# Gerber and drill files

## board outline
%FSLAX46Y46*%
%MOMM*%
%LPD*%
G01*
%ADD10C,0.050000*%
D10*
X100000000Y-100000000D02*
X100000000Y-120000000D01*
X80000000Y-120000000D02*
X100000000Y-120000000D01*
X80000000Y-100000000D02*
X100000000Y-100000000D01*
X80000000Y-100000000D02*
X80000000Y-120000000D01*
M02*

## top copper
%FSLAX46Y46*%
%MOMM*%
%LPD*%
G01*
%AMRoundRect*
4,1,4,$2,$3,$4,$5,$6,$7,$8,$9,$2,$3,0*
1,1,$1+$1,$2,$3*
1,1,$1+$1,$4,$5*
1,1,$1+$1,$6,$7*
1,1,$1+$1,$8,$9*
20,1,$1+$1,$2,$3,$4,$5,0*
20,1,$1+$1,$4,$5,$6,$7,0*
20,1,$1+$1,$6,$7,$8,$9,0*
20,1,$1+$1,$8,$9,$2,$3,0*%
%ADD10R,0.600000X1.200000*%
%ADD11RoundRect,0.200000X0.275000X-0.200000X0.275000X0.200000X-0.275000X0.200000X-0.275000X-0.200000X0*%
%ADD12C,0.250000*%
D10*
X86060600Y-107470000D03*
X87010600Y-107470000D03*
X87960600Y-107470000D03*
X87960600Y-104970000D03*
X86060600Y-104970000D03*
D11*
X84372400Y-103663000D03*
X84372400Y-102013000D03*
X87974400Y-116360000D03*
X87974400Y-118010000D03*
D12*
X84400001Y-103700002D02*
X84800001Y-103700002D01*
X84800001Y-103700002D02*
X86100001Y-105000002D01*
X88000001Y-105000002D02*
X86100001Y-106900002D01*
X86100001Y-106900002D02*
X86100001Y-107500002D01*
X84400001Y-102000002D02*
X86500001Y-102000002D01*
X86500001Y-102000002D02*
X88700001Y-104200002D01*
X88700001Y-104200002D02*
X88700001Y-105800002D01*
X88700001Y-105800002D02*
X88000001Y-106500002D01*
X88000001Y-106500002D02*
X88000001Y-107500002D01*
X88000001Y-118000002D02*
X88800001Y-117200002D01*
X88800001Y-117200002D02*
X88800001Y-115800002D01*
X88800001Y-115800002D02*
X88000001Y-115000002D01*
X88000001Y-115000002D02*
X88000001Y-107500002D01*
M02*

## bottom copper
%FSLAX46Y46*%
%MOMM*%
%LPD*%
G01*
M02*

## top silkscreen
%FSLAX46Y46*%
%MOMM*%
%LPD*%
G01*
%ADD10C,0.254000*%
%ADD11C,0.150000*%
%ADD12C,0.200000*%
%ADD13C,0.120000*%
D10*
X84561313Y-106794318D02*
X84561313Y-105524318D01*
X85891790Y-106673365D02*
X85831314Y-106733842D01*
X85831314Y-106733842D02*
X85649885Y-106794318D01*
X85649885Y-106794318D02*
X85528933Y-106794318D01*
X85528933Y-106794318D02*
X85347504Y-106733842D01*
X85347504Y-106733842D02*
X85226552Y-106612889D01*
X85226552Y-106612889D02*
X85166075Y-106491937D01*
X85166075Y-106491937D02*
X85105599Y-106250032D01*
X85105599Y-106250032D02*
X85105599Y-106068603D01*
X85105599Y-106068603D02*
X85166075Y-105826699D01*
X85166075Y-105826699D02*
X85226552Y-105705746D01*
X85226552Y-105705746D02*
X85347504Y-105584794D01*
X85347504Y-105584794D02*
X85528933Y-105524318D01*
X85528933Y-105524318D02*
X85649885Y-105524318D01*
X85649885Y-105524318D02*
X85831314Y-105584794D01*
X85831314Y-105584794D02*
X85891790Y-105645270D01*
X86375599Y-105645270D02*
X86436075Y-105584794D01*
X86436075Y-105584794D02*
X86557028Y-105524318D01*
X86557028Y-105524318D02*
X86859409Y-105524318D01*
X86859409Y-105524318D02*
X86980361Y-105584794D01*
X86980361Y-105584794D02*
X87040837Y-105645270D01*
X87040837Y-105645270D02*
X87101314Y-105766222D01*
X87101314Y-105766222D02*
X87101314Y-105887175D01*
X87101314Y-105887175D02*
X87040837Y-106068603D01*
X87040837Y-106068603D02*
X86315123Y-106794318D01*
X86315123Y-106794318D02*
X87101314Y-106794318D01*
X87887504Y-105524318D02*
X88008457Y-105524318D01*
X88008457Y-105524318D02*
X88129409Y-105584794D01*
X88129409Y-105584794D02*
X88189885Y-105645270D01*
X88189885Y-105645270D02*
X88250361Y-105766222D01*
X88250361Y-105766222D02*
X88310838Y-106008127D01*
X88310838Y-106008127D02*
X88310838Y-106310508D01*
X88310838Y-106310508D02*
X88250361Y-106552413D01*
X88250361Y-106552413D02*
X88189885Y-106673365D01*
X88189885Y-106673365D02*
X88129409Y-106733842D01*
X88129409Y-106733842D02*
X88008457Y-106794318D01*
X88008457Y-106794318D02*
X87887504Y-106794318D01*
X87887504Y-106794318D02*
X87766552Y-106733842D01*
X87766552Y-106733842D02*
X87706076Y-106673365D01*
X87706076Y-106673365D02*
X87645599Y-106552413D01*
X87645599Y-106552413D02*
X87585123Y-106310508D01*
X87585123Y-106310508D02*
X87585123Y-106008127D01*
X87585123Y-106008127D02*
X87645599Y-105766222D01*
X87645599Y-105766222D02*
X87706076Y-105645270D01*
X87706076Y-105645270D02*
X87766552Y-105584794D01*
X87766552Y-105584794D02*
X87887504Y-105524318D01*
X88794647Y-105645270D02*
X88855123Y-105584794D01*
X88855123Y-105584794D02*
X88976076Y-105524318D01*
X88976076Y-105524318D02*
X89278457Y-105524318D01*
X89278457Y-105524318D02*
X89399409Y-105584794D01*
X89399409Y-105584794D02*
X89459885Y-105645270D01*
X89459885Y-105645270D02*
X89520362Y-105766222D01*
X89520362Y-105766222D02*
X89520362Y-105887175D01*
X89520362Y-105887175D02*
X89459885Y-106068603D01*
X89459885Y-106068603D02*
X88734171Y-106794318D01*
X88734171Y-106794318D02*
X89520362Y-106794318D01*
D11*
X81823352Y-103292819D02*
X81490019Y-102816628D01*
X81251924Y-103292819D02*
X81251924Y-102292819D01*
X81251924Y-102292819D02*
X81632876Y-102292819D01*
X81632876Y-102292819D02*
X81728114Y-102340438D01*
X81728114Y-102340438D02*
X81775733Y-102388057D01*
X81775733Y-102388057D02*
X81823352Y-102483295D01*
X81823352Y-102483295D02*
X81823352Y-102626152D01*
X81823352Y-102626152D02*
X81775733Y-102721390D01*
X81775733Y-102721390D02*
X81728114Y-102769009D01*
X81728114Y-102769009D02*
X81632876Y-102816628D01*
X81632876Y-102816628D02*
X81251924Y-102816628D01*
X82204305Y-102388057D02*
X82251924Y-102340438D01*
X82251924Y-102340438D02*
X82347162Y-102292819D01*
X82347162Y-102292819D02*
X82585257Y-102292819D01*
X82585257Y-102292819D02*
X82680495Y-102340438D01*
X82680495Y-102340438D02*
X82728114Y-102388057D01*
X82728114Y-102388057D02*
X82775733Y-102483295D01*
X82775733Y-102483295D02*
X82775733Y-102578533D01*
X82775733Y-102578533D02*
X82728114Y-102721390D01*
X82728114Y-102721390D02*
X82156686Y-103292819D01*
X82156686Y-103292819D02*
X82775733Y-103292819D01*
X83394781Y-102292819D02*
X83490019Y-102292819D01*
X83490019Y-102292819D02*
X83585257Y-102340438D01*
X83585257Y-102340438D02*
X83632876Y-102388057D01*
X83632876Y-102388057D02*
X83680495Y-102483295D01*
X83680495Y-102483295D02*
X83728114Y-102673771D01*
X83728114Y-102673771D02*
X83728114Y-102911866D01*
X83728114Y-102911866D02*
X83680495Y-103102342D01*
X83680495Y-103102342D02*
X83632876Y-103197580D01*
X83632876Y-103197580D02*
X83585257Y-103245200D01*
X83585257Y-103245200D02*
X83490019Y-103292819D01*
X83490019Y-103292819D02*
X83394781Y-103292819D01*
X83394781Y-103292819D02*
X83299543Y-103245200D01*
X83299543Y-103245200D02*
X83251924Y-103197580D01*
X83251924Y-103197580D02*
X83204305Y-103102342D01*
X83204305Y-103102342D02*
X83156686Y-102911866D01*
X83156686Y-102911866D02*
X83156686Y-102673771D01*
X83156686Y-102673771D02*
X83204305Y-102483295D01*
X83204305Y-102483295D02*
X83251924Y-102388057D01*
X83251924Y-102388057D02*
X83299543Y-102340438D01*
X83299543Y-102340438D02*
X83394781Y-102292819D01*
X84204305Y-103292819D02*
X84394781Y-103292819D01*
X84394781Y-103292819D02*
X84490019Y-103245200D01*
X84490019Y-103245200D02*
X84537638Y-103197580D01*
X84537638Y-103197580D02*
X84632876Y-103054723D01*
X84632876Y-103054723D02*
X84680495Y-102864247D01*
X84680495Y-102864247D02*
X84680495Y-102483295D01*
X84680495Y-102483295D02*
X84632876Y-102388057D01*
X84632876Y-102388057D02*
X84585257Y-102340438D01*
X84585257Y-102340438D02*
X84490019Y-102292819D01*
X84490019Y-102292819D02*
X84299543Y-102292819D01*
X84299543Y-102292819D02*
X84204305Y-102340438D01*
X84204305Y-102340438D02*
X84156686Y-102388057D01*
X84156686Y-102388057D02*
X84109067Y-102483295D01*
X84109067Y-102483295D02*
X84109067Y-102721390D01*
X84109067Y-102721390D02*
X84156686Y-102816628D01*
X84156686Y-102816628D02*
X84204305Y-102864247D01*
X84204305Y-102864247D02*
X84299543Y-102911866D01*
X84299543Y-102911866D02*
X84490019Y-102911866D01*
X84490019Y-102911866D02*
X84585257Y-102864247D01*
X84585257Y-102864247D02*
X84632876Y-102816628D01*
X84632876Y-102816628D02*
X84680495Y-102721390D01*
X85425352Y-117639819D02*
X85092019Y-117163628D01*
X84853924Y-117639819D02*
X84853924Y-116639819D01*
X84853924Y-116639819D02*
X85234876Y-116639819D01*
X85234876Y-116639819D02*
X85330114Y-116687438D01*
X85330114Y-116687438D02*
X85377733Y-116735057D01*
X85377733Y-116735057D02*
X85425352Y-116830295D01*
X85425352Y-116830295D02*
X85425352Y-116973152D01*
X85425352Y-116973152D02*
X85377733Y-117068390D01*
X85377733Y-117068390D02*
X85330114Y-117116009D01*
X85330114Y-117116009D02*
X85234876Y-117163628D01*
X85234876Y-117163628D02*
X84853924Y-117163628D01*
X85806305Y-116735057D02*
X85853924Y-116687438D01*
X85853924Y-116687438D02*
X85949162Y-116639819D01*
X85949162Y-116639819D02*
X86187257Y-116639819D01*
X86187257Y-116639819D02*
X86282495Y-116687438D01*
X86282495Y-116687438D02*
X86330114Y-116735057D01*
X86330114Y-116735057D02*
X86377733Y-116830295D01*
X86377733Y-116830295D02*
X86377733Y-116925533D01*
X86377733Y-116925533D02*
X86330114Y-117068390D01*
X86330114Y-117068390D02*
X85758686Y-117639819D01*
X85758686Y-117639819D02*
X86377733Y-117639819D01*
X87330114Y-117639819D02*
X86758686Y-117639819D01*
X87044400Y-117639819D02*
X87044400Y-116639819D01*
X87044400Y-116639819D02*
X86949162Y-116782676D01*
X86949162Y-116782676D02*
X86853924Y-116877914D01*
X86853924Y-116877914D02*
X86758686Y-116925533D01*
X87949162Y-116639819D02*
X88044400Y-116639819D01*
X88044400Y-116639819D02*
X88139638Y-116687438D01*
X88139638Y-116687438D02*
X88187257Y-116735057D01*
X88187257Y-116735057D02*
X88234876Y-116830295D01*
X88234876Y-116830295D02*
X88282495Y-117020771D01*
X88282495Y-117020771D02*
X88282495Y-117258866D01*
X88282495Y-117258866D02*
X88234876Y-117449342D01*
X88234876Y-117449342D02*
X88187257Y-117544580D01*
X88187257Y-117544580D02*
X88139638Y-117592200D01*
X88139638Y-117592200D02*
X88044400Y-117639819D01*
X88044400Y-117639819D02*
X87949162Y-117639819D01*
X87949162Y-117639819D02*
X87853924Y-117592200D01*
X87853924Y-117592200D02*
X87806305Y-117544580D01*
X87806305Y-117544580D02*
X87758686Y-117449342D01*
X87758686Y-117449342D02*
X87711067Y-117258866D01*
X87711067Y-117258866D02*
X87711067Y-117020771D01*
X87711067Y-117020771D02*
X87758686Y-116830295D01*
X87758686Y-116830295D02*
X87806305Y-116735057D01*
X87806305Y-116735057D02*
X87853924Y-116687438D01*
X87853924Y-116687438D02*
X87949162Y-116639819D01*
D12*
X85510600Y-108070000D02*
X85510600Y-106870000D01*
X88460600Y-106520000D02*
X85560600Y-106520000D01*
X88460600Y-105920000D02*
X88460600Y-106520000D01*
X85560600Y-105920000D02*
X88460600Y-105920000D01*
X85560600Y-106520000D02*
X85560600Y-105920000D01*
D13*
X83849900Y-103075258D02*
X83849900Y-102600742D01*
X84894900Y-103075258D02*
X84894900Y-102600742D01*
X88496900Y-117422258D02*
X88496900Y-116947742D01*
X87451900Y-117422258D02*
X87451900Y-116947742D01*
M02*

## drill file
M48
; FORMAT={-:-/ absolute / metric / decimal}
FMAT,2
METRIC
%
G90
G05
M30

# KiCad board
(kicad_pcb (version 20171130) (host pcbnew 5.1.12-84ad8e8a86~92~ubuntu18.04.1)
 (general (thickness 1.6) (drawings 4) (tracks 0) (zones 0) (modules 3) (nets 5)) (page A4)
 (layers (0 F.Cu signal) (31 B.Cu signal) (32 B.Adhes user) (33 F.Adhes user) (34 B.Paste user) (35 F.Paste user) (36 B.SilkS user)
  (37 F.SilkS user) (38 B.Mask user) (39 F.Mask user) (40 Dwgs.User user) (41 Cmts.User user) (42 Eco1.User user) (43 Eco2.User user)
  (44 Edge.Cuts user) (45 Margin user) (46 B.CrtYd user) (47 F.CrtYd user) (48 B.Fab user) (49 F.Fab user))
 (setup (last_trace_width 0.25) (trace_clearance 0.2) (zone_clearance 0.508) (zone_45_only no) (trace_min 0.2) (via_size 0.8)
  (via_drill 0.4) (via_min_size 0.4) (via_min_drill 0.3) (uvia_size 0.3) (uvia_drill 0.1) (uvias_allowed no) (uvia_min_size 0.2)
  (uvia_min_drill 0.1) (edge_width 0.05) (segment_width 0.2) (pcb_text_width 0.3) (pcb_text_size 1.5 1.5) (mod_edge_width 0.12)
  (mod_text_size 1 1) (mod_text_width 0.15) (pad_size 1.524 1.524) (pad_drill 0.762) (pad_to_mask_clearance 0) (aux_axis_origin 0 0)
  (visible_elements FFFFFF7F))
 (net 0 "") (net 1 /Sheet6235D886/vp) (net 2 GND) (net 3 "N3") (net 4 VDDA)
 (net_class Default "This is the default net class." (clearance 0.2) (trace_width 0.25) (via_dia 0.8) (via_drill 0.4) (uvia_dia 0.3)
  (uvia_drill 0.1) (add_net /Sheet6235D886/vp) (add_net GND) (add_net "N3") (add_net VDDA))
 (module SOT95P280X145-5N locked (layer F.Cu) (at 87.010600 106.220000 90.000000)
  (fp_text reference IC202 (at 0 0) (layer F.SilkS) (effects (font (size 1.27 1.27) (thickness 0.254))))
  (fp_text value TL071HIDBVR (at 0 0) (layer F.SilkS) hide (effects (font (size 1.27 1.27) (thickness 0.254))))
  (fp_line (start -1.85 -1.5) (end -0.65 -1.5) (layer F.SilkS) (width 0.2))
  (fp_line (start -0.3 1.45) (end -0.3 -1.45) (layer F.SilkS) (width 0.2))
  (fp_line (start 0.3 1.45) (end -0.3 1.45) (layer F.SilkS) (width 0.2))
  (fp_line (start 0.3 -1.45) (end 0.3 1.45) (layer F.SilkS) (width 0.2))
  (fp_line (start -0.3 -1.45) (end 0.3 -1.45) (layer F.SilkS) (width 0.2))
  (pad 1 smd rect (at -1.25 -0.95 180.000000) (size 0.6 1.2) (layers F.Cu F.Mask F.Paste) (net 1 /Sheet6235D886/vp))
  (pad 2 smd rect (at -1.25 0 180.000000) (size 0.6 1.2) (layers F.Cu F.Mask F.Paste) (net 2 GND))
  (pad 3 smd rect (at -1.25 0.95 180.000000) (size 0.6 1.2) (layers F.Cu F.Mask F.Paste) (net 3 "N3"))
  (pad 4 smd rect (at 1.25 0.95 180.000000) (size 0.6 1.2) (layers F.Cu F.Mask F.Paste) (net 1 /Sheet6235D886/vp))
  (pad 5 smd rect (at 1.25 -0.95 180.000000) (size 0.6 1.2) (layers F.Cu F.Mask F.Paste) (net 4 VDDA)))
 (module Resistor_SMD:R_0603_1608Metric (layer F.Cu) (at 84.372400 102.838000 90.000000)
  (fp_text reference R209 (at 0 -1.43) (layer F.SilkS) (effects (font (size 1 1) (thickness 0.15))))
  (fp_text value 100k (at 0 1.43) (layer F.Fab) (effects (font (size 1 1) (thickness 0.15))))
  (fp_line (start -0.237258 -0.5225) (end 0.237258 -0.5225) (layer F.SilkS) (width 0.12))
  (fp_line (start -0.237258 0.5225) (end 0.237258 0.5225) (layer F.SilkS) (width 0.12))
  (pad 1 smd roundrect (at -0.825 0 90.000000) (size 0.8 0.95) (layers F.Cu F.Mask F.Paste) (roundrect_rratio 0.25) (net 4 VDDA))
  (pad 2 smd roundrect (at 0.825 0 90.000000) (size 0.8 0.95) (layers F.Cu F.Mask F.Paste) (roundrect_rratio 0.25) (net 3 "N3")))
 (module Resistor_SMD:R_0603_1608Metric (layer F.Cu) (at 87.974400 117.185000 90.000000)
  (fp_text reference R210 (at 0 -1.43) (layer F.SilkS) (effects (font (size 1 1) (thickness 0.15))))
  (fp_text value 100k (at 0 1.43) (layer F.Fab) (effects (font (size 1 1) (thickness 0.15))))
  (fp_line (start -0.237258 0.5225) (end 0.237258 0.5225) (layer F.SilkS) (width 0.12))
  (fp_line (start -0.237258 -0.5225) (end 0.237258 -0.5225) (layer F.SilkS) (width 0.12))
  (pad 2 smd roundrect (at 0.825 0 90.000000) (size 0.8 0.95) (layers F.Cu F.Mask F.Paste) (roundrect_rratio 0.25) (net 2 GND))
  (pad 1 smd roundrect (at -0.825 0 90.000000) (size 0.8 0.95) (layers F.Cu F.Mask F.Paste) (roundrect_rratio 0.25) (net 3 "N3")))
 (gr_line (start 100 100) (end 100 120) (layer Edge.Cuts) (width 0.05))
 (gr_line (start 80 120) (end 100 120) (layer Edge.Cuts) (width 0.05))
 (gr_line (start 80 100) (end 100 100) (layer Edge.Cuts) (width 0.05))
 (gr_line (start 80 100) (end 80 120) (layer Edge.Cuts) (width 0.05))
 (segment (start 84.400001 103.700002) (end 84.800001 103.700002) (width 0.250000) (layer F.Cu) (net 4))
 (segment (start 84.800001 103.700002) (end 86.100001 105.000002) (width 0.250000) (layer F.Cu) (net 4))
 (segment (start 88.000001 105.000002) (end 86.100001 106.900002) (width 0.250000) (layer F.Cu) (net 1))
 (segment (start 86.100001 106.900002) (end 86.100001 107.500002) (width 0.250000) (layer F.Cu) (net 1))
 (segment (start 84.400001 102.000002) (end 86.500001 102.000002) (width 0.250000) (layer F.Cu) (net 3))
 (segment (start 86.500001 102.000002) (end 88.700001 104.200002) (width 0.250000) (layer F.Cu) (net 3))
 (segment (start 88.700001 104.200002) (end 88.700001 105.800002) (width 0.250000) (layer F.Cu) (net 3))
 (segment (start 88.700001 105.800002) (end 88.000001 106.500002) (width 0.250000) (layer F.Cu) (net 3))
 (segment (start 88.000001 106.500002) (end 88.000001 107.500002) (width 0.250000) (layer F.Cu) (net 3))
 (segment (start 88.000001 118.000002) (end 88.800001 117.200002) (width 0.250000) (layer F.Cu) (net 3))
 (segment (start 88.800001 117.200002) (end 88.800001 115.800002) (width 0.250000) (layer F.Cu) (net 3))
 (segment (start 88.800001 115.800002) (end 88.000001 115.000002) (width 0.250000) (layer F.Cu) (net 3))
 (segment (start 88.000001 115.000002) (end 88.000001 107.500002) (width 0.250000) (layer F.Cu) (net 3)))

